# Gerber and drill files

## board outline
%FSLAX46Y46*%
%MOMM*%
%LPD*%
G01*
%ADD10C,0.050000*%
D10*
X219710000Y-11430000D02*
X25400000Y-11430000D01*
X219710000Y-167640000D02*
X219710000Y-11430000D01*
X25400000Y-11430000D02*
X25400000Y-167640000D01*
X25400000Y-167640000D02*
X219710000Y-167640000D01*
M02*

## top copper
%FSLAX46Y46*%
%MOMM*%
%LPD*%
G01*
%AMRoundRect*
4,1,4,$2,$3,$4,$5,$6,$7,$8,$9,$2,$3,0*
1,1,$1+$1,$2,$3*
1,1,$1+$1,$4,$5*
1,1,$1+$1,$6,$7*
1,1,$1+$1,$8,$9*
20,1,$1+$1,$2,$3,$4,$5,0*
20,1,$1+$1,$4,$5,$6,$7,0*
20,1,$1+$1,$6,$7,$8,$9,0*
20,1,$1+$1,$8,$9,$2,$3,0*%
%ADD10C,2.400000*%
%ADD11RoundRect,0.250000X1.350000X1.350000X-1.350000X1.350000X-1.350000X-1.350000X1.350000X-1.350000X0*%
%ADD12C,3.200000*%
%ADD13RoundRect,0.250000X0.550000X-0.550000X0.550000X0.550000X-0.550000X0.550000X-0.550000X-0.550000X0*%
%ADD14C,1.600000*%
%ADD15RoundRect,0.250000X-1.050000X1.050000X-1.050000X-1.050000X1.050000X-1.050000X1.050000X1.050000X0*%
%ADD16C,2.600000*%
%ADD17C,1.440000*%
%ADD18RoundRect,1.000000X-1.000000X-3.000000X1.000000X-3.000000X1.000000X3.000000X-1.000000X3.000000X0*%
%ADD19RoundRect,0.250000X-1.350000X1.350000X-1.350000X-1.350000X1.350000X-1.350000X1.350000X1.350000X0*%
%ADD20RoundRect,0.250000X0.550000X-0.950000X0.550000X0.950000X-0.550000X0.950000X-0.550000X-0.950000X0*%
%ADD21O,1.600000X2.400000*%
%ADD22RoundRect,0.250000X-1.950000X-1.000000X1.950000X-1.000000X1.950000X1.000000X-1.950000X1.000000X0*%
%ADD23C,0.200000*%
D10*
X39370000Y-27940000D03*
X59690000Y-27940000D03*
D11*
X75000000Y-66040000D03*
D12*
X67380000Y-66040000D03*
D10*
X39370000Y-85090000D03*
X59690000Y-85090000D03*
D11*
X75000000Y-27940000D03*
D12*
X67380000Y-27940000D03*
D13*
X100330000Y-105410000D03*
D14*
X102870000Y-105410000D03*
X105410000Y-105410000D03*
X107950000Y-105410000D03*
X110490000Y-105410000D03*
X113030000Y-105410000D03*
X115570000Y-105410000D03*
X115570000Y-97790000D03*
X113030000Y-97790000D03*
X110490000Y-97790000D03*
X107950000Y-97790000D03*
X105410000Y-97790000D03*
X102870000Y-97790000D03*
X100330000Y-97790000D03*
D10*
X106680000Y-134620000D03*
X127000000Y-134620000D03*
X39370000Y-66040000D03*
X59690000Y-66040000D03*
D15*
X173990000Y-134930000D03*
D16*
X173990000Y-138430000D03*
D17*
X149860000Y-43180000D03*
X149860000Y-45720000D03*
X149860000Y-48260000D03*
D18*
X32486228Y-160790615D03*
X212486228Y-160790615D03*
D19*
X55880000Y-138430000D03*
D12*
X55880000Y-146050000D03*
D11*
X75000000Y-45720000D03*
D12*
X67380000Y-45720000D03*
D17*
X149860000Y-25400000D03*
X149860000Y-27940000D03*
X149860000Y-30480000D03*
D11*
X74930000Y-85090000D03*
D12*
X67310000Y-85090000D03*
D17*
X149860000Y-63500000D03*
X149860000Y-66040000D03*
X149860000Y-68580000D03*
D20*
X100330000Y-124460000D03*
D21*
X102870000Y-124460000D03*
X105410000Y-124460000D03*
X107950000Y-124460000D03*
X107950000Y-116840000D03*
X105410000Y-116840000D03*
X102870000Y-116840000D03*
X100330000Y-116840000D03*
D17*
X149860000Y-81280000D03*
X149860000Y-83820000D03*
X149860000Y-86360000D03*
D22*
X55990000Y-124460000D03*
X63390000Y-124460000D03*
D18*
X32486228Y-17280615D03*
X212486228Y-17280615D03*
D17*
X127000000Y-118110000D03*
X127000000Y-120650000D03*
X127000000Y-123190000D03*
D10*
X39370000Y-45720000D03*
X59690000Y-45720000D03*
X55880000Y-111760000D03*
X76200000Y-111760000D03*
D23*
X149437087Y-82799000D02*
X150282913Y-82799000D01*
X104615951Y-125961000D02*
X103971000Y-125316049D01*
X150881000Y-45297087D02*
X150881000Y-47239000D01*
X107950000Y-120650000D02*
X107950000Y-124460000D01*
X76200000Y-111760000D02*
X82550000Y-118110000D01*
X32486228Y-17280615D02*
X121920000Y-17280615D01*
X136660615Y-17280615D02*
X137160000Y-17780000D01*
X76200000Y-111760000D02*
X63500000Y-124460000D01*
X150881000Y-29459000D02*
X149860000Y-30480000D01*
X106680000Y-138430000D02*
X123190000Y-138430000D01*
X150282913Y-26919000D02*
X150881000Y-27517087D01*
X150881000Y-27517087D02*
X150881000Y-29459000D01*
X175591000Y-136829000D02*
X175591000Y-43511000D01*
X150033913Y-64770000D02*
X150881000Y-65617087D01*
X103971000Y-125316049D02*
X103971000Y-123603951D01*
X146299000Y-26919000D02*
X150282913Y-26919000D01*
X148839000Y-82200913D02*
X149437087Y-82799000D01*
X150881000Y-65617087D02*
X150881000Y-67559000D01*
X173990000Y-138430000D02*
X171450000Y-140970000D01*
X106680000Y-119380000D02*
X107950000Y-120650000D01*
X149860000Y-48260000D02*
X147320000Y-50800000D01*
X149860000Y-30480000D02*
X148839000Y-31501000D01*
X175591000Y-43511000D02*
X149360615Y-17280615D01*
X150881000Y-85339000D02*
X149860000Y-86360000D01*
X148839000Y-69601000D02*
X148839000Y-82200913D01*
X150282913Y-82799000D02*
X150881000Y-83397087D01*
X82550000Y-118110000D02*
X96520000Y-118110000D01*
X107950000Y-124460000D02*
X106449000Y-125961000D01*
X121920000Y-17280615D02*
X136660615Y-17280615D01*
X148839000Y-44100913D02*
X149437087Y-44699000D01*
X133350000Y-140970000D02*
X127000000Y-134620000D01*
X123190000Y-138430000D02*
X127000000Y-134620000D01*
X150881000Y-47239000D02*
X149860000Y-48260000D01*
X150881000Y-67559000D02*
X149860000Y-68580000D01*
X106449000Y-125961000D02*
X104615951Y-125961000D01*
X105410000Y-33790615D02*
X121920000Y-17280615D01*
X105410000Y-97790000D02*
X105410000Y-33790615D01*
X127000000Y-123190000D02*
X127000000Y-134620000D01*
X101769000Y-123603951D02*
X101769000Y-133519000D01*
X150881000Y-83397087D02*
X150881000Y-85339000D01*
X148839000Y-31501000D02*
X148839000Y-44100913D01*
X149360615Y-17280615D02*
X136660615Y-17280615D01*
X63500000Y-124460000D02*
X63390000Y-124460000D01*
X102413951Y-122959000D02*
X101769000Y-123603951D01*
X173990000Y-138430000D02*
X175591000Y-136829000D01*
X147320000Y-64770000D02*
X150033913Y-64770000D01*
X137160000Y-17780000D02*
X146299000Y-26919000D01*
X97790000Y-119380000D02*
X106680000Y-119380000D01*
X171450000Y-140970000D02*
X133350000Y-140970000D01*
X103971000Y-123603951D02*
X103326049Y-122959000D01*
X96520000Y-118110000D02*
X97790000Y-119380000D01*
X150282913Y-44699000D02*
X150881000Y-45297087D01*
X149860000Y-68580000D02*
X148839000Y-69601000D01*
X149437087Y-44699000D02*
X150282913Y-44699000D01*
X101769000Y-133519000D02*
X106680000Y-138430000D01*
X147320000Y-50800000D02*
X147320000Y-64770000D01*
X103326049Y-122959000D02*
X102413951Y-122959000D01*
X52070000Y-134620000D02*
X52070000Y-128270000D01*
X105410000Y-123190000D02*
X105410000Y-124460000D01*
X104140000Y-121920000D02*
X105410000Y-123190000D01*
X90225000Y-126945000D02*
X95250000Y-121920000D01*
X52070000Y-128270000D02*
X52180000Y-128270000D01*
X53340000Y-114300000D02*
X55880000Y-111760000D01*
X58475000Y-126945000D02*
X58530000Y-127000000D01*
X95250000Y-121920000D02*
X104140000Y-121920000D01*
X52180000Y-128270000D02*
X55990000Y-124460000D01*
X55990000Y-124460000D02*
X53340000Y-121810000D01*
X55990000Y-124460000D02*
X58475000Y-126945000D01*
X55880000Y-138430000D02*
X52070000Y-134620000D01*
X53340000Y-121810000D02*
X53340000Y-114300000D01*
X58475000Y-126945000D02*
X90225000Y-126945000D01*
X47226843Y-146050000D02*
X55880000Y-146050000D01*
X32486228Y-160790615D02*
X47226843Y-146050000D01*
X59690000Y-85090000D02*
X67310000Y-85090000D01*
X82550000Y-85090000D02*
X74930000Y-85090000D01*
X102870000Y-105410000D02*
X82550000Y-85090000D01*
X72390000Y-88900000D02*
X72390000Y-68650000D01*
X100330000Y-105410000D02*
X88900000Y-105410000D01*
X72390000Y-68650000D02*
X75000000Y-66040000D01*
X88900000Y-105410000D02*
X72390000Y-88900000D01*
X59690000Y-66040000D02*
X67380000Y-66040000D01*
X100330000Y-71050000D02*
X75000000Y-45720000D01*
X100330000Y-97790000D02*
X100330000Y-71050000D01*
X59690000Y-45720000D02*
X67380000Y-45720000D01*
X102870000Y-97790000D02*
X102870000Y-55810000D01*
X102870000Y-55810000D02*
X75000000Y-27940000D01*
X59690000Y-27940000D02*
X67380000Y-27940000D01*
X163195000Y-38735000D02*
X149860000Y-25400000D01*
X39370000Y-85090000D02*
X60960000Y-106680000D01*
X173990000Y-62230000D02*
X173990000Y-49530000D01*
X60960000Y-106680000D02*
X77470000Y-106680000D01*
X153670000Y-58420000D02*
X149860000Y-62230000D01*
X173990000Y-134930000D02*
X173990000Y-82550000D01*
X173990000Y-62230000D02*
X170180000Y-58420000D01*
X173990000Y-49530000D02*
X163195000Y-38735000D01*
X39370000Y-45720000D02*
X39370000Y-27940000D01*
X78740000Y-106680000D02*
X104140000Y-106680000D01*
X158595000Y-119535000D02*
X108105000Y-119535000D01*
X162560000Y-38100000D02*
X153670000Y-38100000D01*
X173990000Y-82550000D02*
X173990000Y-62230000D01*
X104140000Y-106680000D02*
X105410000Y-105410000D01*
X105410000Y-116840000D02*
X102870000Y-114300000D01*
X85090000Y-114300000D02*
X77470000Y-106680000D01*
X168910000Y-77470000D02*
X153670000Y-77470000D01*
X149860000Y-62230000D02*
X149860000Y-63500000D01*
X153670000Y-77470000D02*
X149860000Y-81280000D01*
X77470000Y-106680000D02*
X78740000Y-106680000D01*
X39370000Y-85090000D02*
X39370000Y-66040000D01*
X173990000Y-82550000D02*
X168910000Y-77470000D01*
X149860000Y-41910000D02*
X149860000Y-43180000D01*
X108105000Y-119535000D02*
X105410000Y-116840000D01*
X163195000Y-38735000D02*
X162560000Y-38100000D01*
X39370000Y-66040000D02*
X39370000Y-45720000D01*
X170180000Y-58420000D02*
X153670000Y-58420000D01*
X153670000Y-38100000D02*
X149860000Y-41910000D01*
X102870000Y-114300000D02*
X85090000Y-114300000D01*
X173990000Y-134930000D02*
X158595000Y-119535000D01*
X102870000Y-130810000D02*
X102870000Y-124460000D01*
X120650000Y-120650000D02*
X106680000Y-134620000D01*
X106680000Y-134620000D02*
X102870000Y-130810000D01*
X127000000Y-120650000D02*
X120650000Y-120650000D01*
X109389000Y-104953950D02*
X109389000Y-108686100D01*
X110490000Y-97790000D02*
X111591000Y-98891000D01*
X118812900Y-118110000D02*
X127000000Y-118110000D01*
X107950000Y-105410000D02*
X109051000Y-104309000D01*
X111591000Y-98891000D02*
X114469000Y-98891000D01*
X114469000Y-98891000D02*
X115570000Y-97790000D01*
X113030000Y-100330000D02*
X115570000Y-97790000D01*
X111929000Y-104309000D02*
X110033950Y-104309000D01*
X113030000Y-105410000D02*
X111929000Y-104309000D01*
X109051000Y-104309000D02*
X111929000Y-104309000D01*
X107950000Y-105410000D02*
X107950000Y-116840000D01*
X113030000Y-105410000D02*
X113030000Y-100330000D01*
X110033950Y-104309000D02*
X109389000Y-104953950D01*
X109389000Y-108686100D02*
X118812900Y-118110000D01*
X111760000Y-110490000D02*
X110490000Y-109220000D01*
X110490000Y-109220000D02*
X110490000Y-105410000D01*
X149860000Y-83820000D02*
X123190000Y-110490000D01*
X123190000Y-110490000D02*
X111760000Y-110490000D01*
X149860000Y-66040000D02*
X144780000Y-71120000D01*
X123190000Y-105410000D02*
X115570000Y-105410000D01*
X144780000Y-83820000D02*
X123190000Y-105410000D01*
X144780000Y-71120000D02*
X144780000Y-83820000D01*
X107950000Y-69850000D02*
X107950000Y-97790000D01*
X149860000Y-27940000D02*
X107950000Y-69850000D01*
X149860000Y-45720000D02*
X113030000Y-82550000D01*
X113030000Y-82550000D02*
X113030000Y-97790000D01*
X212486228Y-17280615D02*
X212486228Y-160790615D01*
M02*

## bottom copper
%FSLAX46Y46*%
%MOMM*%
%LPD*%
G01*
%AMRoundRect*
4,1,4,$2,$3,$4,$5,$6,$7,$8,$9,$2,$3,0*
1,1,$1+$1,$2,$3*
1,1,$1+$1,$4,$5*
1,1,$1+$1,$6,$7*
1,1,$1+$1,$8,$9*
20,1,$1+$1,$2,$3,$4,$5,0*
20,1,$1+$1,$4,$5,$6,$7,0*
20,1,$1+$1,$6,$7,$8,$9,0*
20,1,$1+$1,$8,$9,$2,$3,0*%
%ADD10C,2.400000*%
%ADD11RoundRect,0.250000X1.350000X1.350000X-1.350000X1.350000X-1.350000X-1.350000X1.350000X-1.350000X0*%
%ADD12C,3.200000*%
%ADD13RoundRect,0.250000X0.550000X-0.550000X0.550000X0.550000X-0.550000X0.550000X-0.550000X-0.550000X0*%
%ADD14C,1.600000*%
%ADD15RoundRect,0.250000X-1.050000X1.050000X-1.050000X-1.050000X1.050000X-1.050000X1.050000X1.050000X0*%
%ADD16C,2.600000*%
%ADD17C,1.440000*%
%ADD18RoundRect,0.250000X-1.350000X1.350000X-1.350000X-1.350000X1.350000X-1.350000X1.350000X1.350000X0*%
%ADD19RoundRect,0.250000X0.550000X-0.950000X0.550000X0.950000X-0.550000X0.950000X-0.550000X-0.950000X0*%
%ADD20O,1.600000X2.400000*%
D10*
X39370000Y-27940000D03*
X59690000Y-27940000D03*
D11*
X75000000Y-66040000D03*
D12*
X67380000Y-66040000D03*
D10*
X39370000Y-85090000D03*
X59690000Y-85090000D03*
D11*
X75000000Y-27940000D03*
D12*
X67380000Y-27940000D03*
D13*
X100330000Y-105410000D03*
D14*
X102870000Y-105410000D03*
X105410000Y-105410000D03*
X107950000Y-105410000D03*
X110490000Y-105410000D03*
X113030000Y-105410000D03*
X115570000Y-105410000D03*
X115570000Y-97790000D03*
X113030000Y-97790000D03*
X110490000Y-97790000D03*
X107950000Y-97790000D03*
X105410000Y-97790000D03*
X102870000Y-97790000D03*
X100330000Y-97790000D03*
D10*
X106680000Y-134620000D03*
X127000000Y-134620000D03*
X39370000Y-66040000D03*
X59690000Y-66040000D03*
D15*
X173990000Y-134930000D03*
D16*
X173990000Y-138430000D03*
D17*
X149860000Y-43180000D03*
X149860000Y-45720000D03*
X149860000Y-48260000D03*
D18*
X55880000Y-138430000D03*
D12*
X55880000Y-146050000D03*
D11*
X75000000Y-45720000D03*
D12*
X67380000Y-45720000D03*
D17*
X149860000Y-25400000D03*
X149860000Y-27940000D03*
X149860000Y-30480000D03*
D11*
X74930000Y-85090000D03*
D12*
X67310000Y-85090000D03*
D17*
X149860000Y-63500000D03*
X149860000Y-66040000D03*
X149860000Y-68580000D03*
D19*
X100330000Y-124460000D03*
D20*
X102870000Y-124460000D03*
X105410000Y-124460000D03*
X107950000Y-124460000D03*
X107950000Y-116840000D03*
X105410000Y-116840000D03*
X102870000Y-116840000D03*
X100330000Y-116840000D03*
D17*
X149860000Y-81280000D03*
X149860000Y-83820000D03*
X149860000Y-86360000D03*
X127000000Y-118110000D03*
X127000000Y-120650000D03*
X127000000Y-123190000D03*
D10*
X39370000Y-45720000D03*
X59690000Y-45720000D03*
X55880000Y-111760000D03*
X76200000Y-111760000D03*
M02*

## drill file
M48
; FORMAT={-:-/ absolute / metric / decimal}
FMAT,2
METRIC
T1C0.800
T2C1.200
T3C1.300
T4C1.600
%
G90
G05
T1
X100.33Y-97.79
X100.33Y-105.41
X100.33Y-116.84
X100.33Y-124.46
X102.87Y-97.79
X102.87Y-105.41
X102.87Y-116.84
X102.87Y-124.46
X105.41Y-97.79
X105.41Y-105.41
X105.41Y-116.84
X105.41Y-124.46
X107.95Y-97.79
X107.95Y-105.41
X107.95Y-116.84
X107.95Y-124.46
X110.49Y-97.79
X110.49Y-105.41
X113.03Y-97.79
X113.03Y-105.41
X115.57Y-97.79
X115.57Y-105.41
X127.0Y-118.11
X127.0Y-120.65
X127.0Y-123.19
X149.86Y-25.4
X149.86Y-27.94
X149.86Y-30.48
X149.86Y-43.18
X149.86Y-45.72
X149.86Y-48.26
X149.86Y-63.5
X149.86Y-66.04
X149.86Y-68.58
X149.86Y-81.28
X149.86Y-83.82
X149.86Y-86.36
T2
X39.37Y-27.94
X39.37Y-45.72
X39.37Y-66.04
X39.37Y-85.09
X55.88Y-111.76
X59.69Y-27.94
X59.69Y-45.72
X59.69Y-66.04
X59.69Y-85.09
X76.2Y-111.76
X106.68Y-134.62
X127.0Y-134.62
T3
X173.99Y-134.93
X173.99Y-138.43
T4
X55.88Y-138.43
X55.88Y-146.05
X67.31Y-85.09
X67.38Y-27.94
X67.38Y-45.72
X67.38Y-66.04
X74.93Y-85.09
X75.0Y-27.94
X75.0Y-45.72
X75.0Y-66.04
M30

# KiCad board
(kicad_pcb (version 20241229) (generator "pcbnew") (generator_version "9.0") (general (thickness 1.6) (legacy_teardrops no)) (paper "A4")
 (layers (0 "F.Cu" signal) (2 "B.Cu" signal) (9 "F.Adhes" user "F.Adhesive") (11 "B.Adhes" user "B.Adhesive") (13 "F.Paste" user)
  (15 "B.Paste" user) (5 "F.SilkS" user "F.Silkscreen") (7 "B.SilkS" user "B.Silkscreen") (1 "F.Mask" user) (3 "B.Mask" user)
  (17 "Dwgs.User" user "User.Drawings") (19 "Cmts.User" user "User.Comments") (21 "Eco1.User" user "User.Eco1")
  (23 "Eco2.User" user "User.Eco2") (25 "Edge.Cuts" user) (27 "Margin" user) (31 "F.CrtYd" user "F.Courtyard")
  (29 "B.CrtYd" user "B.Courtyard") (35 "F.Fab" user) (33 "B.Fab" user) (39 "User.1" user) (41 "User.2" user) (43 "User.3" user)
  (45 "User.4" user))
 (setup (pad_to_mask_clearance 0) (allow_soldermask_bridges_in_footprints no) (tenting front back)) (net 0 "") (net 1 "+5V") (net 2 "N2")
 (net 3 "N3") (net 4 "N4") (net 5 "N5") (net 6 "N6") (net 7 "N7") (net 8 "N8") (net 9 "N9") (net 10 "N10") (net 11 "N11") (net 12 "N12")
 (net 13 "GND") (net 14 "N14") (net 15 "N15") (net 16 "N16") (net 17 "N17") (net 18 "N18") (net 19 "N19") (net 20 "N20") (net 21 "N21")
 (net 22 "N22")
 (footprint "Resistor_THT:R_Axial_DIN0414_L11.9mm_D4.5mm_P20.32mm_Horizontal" (layer "F.Cu") (at 39.37 27.94)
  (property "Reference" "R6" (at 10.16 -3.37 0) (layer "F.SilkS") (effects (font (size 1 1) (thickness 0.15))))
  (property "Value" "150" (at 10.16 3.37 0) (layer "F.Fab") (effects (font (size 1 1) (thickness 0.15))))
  (pad "1" thru_hole circle (at 0 0) (size 2.4 2.4) (drill 1.2) (layers "*.Cu" "*.Mask") (remove_unused_layers no) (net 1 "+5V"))
  (pad "2" thru_hole circle (at 20.32 0) (size 2.4 2.4) (drill 1.2) (layers "*.Cu" "*.Mask") (remove_unused_layers no) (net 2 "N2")))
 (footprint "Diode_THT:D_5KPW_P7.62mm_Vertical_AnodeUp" (layer "F.Cu") (at 75 66.04 180)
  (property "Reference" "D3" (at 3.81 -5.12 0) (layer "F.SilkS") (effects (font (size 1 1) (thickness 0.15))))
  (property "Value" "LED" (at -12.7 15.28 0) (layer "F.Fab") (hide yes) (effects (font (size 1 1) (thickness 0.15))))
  (pad "1" thru_hole roundrect (at 0 0 180) (size 3.2 3.2) (drill 1.6) (layers "*.Cu" "*.Mask") (remove_unused_layers no)
   (roundrect_rratio 0.078125) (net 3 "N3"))
  (pad "2" thru_hole circle (at 7.62 0 180) (size 3.2 3.2) (drill 1.6) (layers "*.Cu" "*.Mask") (remove_unused_layers no) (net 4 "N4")))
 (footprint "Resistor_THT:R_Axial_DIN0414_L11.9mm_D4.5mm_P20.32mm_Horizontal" (layer "F.Cu") (at 39.37 85.09)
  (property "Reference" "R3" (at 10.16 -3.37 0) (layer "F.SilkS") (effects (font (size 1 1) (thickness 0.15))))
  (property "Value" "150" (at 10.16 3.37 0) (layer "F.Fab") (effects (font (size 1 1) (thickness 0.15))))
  (pad "1" thru_hole circle (at 0 0) (size 2.4 2.4) (drill 1.2) (layers "*.Cu" "*.Mask") (remove_unused_layers no) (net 1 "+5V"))
  (pad "2" thru_hole circle (at 20.32 0) (size 2.4 2.4) (drill 1.2) (layers "*.Cu" "*.Mask") (remove_unused_layers no) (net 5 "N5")))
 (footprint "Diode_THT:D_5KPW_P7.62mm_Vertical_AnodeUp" (layer "F.Cu") (at 75 27.94 180)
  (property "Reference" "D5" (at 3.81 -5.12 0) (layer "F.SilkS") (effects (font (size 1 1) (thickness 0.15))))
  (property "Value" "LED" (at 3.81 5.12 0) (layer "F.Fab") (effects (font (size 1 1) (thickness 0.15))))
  (pad "1" thru_hole roundrect (at 0 0 180) (size 3.2 3.2) (drill 1.6) (layers "*.Cu" "*.Mask") (remove_unused_layers no)
   (roundrect_rratio 0.078125) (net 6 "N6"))
  (pad "2" thru_hole circle (at 7.62 0 180) (size 3.2 3.2) (drill 1.6) (layers "*.Cu" "*.Mask") (remove_unused_layers no) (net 2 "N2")))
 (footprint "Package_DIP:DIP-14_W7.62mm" (layer "F.Cu") (at 100.33 105.41 90)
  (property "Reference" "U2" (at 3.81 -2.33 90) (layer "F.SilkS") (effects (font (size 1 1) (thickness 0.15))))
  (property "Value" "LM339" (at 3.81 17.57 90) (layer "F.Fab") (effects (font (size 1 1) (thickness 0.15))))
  (pad "1" thru_hole roundrect (at 0 0 90) (size 1.6 1.6) (drill 0.8) (layers "*.Cu" "*.Mask") (remove_unused_layers no)
   (roundrect_rratio 0.15625) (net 3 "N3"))
  (pad "2" thru_hole circle (at 0 2.54 90) (size 1.6 1.6) (drill 0.8) (layers "*.Cu" "*.Mask") (remove_unused_layers no) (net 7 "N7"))
  (pad "3" thru_hole circle (at 0 5.08 90) (size 1.6 1.6) (drill 0.8) (layers "*.Cu" "*.Mask") (remove_unused_layers no) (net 1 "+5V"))
  (pad "4" thru_hole circle (at 0 7.62 90) (size 1.6 1.6) (drill 0.8) (layers "*.Cu" "*.Mask") (remove_unused_layers no) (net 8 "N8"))
  (pad "5" thru_hole circle (at 0 10.16 90) (size 1.6 1.6) (drill 0.8) (layers "*.Cu" "*.Mask") (remove_unused_layers no) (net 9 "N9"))
  (pad "6" thru_hole circle (at 0 12.7 90) (size 1.6 1.6) (drill 0.8) (layers "*.Cu" "*.Mask") (remove_unused_layers no) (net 8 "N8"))
  (pad "7" thru_hole circle (at 0 15.24 90) (size 1.6 1.6) (drill 0.8) (layers "*.Cu" "*.Mask") (remove_unused_layers no) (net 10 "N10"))
  (pad "8" thru_hole circle (at 7.62 15.24 90) (size 1.6 1.6) (drill 0.8) (layers "*.Cu" "*.Mask") (remove_unused_layers no) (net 8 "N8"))
  (pad "9" thru_hole circle (at 7.62 12.7 90) (size 1.6 1.6) (drill 0.8) (layers "*.Cu" "*.Mask") (remove_unused_layers no) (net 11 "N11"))
  (pad "10" thru_hole circle (at 7.62 10.16 90) (size 1.6 1.6) (drill 0.8) (layers "*.Cu" "*.Mask") (remove_unused_layers no) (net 8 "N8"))
  (pad "11" thru_hole circle (at 7.62 7.62 90) (size 1.6 1.6) (drill 0.8) (layers "*.Cu" "*.Mask") (remove_unused_layers no) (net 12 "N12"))
  (pad "12" thru_hole circle (at 7.62 5.08 90) (size 1.6 1.6) (drill 0.8) (layers "*.Cu" "*.Mask") (remove_unused_layers no) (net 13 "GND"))
  (pad "13" thru_hole circle (at 7.62 2.54 90) (size 1.6 1.6) (drill 0.8) (layers "*.Cu" "*.Mask") (remove_unused_layers no) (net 6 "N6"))
  (pad "14" thru_hole circle (at 7.62 0 90) (size 1.6 1.6) (drill 0.8) (layers "*.Cu" "*.Mask") (remove_unused_layers no) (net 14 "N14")))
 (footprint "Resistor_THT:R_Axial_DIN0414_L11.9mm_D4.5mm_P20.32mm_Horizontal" (layer "F.Cu") (at 106.68 134.62)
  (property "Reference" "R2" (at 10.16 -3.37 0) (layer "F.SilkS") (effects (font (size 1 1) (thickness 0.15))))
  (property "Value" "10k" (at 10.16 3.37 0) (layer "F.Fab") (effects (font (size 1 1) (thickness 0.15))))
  (pad "1" thru_hole circle (at 0 0) (size 2.4 2.4) (drill 1.2) (layers "*.Cu" "*.Mask") (remove_unused_layers no) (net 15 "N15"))
  (pad "2" thru_hole circle (at 20.32 0) (size 2.4 2.4) (drill 1.2) (layers "*.Cu" "*.Mask") (remove_unused_layers no) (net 13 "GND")))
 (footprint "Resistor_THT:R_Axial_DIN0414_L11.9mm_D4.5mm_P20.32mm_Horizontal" (layer "F.Cu") (at 39.37 66.04)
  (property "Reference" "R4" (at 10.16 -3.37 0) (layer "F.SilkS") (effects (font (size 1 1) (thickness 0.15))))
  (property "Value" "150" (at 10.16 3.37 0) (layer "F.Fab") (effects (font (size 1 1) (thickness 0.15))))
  (pad "1" thru_hole circle (at 0 0) (size 2.4 2.4) (drill 1.2) (layers "*.Cu" "*.Mask") (remove_unused_layers no) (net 1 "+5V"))
  (pad "2" thru_hole circle (at 20.32 0) (size 2.4 2.4) (drill 1.2) (layers "*.Cu" "*.Mask") (remove_unused_layers no) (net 4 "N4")))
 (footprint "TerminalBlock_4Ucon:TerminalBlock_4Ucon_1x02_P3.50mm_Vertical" (layer "F.Cu") (at 173.99 134.93 -90)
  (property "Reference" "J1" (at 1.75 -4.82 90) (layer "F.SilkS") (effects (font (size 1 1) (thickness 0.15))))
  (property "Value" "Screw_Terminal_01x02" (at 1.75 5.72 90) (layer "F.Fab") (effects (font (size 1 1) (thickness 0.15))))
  (pad "1" thru_hole roundrect (at 0 0 270) (size 2.6 2.6) (drill 1.3) (layers "*.Cu" "*.Mask") (remove_unused_layers no)
   (roundrect_rratio 0.096154) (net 1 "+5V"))
  (pad "2" thru_hole circle (at 3.5 0 270) (size 2.6 2.6) (drill 1.3) (layers "*.Cu" "*.Mask") (remove_unused_layers no) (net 13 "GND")))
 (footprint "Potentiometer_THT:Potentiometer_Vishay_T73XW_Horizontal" (layer "F.Cu") (at 149.86 43.18)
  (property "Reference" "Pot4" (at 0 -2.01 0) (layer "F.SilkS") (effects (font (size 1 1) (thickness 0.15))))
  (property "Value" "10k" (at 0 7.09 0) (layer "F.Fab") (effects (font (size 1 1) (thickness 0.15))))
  (pad "1" thru_hole circle (at 0 0) (size 1.44 1.44) (drill 0.8) (layers "*.Cu" "*.Mask") (remove_unused_layers no) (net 1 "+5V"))
  (pad "2" thru_hole circle (at 0 2.54) (size 1.44 1.44) (drill 0.8) (layers "*.Cu" "*.Mask") (remove_unused_layers no) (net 11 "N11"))
  (pad "3" thru_hole circle (at 0 5.08) (size 1.44 1.44) (drill 0.8) (layers "*.Cu" "*.Mask") (remove_unused_layers no) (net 13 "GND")))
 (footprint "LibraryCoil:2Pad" (layer "F.Cu") (at 32.486228 160.790615 90)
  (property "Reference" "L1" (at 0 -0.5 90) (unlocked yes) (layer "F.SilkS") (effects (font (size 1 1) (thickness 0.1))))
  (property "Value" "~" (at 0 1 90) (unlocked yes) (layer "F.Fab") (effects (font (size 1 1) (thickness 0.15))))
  (pad "1" smd roundrect (at 0 0) (size 4 8) (layers "F.Cu" "F.Mask") (roundrect_rratio 0.25) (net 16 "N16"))
  (pad "2" smd roundrect (at 0 180) (size 4 8) (layers "F.Cu" "F.Mask") (roundrect_rratio 0.25) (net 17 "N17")))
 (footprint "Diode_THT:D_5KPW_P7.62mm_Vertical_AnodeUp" (layer "F.Cu") (at 55.88 138.43 -90)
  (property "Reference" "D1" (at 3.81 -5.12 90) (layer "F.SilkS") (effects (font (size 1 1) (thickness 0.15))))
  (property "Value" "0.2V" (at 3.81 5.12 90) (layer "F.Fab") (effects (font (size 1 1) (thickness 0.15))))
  (pad "1" thru_hole roundrect (at 0 0 270) (size 3.2 3.2) (drill 1.6) (layers "*.Cu" "*.Mask") (remove_unused_layers no)
   (roundrect_rratio 0.078125) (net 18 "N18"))
  (pad "2" thru_hole circle (at 7.62 0 270) (size 3.2 3.2) (drill 1.6) (layers "*.Cu" "*.Mask") (remove_unused_layers no) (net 16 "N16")))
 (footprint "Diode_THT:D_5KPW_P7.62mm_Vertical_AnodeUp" (layer "F.Cu") (at 75 45.72 180)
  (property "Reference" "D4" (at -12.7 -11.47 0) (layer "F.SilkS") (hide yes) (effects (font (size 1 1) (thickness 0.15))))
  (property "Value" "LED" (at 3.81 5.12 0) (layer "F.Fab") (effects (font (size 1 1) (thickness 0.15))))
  (pad "1" thru_hole roundrect (at 0 0 180) (size 3.2 3.2) (drill 1.6) (layers "*.Cu" "*.Mask") (remove_unused_layers no)
   (roundrect_rratio 0.078125) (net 14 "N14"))
  (pad "2" thru_hole circle (at 7.62 0 180) (size 3.2 3.2) (drill 1.6) (layers "*.Cu" "*.Mask") (remove_unused_layers no) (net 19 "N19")))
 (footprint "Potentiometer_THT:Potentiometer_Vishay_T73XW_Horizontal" (layer "F.Cu") (at 149.86 25.4)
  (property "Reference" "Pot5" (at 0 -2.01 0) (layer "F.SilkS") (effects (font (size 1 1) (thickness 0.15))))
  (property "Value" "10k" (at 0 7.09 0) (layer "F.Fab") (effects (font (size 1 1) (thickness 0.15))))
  (pad "1" thru_hole circle (at 0 0) (size 1.44 1.44) (drill 0.8) (layers "*.Cu" "*.Mask") (remove_unused_layers no) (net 1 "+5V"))
  (pad "2" thru_hole circle (at 0 2.54) (size 1.44 1.44) (drill 0.8) (layers "*.Cu" "*.Mask") (remove_unused_layers no) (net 12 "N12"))
  (pad "3" thru_hole circle (at 0 5.08) (size 1.44 1.44) (drill 0.8) (layers "*.Cu" "*.Mask") (remove_unused_layers no) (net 13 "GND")))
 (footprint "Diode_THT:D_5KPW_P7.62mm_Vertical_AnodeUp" (layer "F.Cu") (at 74.93 85.09 180)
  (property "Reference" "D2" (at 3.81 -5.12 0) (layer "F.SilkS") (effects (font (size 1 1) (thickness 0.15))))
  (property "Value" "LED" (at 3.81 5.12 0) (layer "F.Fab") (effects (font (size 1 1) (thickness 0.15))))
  (pad "1" thru_hole roundrect (at 0 0 180) (size 3.2 3.2) (drill 1.6) (layers "*.Cu" "*.Mask") (remove_unused_layers no)
   (roundrect_rratio 0.078125) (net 7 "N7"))
  (pad "2" thru_hole circle (at 7.62 0 180) (size 3.2 3.2) (drill 1.6) (layers "*.Cu" "*.Mask") (remove_unused_layers no) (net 5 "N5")))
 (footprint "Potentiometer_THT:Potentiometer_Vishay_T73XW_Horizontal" (layer "F.Cu") (at 149.86 63.5)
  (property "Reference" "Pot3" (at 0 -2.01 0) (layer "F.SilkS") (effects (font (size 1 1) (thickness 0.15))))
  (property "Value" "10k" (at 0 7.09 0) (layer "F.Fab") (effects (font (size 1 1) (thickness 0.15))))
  (pad "1" thru_hole circle (at 0 0) (size 1.44 1.44) (drill 0.8) (layers "*.Cu" "*.Mask") (remove_unused_layers no) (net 1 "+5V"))
  (pad "2" thru_hole circle (at 0 2.54) (size 1.44 1.44) (drill 0.8) (layers "*.Cu" "*.Mask") (remove_unused_layers no) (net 10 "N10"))
  (pad "3" thru_hole circle (at 0 5.08) (size 1.44 1.44) (drill 0.8) (layers "*.Cu" "*.Mask") (remove_unused_layers no) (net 13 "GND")))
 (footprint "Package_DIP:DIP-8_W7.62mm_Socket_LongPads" (layer "F.Cu") (at 100.33 124.46 90)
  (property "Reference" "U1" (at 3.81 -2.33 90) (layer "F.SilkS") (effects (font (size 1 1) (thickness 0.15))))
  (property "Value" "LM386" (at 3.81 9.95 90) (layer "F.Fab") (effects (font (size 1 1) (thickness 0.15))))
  (pad "1" thru_hole roundrect (at 0 0 90) (size 2.4 1.6) (drill 0.8) (layers "*.Cu" "*.Mask") (remove_unused_layers no)
   (roundrect_rratio 0.15625) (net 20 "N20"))
  (pad "2" thru_hole oval (at 0 2.54 90) (size 2.4 1.6) (drill 0.8) (layers "*.Cu" "*.Mask") (remove_unused_layers no) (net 15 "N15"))
  (pad "3" thru_hole oval (at 0 5.08 90) (size 2.4 1.6) (drill 0.8) (layers "*.Cu" "*.Mask") (remove_unused_layers no) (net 18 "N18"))
  (pad "4" thru_hole oval (at 0 7.62 90) (size 2.4 1.6) (drill 0.8) (layers "*.Cu" "*.Mask") (remove_unused_layers no) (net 13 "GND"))
  (pad "5" thru_hole oval (at 7.62 7.62 90) (size 2.4 1.6) (drill 0.8) (layers "*.Cu" "*.Mask") (remove_unused_layers no) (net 8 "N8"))
  (pad "6" thru_hole oval (at 7.62 5.08 90) (size 2.4 1.6) (drill 0.8) (layers "*.Cu" "*.Mask") (remove_unused_layers no) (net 1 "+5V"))
  (pad "7" thru_hole oval (at 7.62 2.54 90) (size 2.4 1.6) (drill 0.8) (layers "*.Cu" "*.Mask") (remove_unused_layers no) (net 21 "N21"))
  (pad "8" thru_hole oval (at 7.62 0 90) (size 2.4 1.6) (drill 0.8) (layers "*.Cu" "*.Mask") (remove_unused_layers no) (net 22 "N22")))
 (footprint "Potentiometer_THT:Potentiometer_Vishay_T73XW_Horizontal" (layer "F.Cu") (at 149.86 81.28)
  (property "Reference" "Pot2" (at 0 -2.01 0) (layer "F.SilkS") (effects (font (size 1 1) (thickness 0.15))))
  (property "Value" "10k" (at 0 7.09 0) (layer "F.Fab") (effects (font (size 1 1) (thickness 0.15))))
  (pad "1" thru_hole circle (at 0 0) (size 1.44 1.44) (drill 0.8) (layers "*.Cu" "*.Mask") (remove_unused_layers no) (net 1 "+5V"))
  (pad "2" thru_hole circle (at 0 2.54) (size 1.44 1.44) (drill 0.8) (layers "*.Cu" "*.Mask") (remove_unused_layers no) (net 9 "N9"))
  (pad "3" thru_hole circle (at 0 5.08) (size 1.44 1.44) (drill 0.8) (layers "*.Cu" "*.Mask") (remove_unused_layers no) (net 13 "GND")))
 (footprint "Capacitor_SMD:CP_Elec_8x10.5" (layer "F.Cu") (at 59.69 124.46)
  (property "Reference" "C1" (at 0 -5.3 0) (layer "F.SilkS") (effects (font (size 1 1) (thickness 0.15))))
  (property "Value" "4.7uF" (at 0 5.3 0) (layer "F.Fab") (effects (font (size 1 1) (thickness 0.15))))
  (pad "1" smd roundrect (at -3.7 0) (size 4.4 2.5) (layers "F.Cu" "F.Mask" "F.Paste") (roundrect_rratio 0.1) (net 18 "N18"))
  (pad "2" smd roundrect (at 3.7 0) (size 4.4 2.5) (layers "F.Cu" "F.Mask" "F.Paste") (roundrect_rratio 0.1) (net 13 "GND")))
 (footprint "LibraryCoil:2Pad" (layer "F.Cu") (at 32.486228 17.280615 90)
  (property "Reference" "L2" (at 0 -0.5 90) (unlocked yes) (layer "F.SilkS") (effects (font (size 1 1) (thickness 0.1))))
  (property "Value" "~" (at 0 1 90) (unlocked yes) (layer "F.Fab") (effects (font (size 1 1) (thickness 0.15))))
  (pad "1" smd roundrect (at 0 0) (size 4 8) (layers "F.Cu" "F.Mask") (roundrect_rratio 0.25) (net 13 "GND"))
  (pad "2" smd roundrect (at 0 180) (size 4 8) (layers "F.Cu" "F.Mask") (roundrect_rratio 0.25) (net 17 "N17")))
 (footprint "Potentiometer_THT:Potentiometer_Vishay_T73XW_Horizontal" (layer "F.Cu") (at 127 118.11)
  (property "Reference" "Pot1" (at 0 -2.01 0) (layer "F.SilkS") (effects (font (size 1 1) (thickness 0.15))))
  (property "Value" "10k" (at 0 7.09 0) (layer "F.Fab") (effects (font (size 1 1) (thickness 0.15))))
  (pad "1" thru_hole circle (at 0 0) (size 1.44 1.44) (drill 0.8) (layers "*.Cu" "*.Mask") (remove_unused_layers no) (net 8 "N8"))
  (pad "2" thru_hole circle (at 0 2.54) (size 1.44 1.44) (drill 0.8) (layers "*.Cu" "*.Mask") (remove_unused_layers no) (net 15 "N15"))
  (pad "3" thru_hole circle (at 0 5.08) (size 1.44 1.44) (drill 0.8) (layers "*.Cu" "*.Mask") (remove_unused_layers no) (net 13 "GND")))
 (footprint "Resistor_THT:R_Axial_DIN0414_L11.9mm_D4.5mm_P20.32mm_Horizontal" (layer "F.Cu") (at 39.37 45.72)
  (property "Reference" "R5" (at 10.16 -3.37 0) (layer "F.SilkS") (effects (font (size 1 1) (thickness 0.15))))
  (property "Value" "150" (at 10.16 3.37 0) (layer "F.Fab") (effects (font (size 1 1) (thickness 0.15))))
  (pad "1" thru_hole circle (at 0 0) (size 2.4 2.4) (drill 1.2) (layers "*.Cu" "*.Mask") (remove_unused_layers no) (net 1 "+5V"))
  (pad "2" thru_hole circle (at 20.32 0) (size 2.4 2.4) (drill 1.2) (layers "*.Cu" "*.Mask") (remove_unused_layers no) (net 19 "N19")))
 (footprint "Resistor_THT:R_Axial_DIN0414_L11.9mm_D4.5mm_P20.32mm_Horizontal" (layer "F.Cu") (at 55.88 111.76)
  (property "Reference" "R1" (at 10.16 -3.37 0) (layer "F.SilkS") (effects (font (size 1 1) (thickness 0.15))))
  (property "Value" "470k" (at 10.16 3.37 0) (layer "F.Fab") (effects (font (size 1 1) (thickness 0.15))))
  (pad "1" thru_hole circle (at 0 0) (size 2.4 2.4) (drill 1.2) (layers "*.Cu" "*.Mask") (remove_unused_layers no) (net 18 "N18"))
  (pad "2" thru_hole circle (at 20.32 0) (size 2.4 2.4) (drill 1.2) (layers "*.Cu" "*.Mask") (remove_unused_layers no) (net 13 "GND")))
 (gr_line (start 219.71 11.43) (end 25.4 11.43) (stroke (width 0.05) (type default)) (layer "Edge.Cuts"))
 (gr_line (start 219.71 167.64) (end 219.71 11.43) (stroke (width 0.05) (type default)) (layer "Edge.Cuts"))
 (gr_line (start 25.4 11.43) (end 25.4 167.64) (stroke (width 0.05) (type default)) (layer "Edge.Cuts"))
 (gr_line (start 25.4 167.64) (end 219.71 167.64) (stroke (width 0.05) (type default)) (layer "Edge.Cuts"))
 (segment (start 149.437087 82.799) (end 150.282913 82.799) (width 0.2) (layer "F.Cu") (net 13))
 (segment (start 104.615951 125.961) (end 103.971 125.316049) (width 0.2) (layer "F.Cu") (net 13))
 (segment (start 150.881 45.297087) (end 150.881 47.239) (width 0.2) (layer "F.Cu") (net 13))
 (segment (start 107.95 120.65) (end 107.95 124.46) (width 0.2) (layer "F.Cu") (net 13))
 (segment (start 76.2 111.76) (end 82.55 118.11) (width 0.2) (layer "F.Cu") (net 13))
 (segment (start 32.486228 17.280615) (end 121.92 17.280615) (width 0.2) (layer "F.Cu") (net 13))
 (segment (start 136.660615 17.280615) (end 137.16 17.78) (width 0.2) (layer "F.Cu") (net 13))
 (segment (start 76.2 111.76) (end 63.5 124.46) (width 0.2) (layer "F.Cu") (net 13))
 (segment (start 150.881 29.459) (end 149.86 30.48) (width 0.2) (layer "F.Cu") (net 13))
 (segment (start 106.68 138.43) (end 123.19 138.43) (width 0.2) (layer "F.Cu") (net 13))
 (segment (start 150.282913 26.919) (end 150.881 27.517087) (width 0.2) (layer "F.Cu") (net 13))
 (segment (start 150.881 27.517087) (end 150.881 29.459) (width 0.2) (layer "F.Cu") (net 13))
 (segment (start 175.591 136.829) (end 175.591 43.511) (width 0.2) (layer "F.Cu") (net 13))
 (segment (start 150.033913 64.77) (end 150.881 65.617087) (width 0.2) (layer "F.Cu") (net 13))
 (segment (start 103.971 125.316049) (end 103.971 123.603951) (width 0.2) (layer "F.Cu") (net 13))
 (segment (start 146.299 26.919) (end 150.282913 26.919) (width 0.2) (layer "F.Cu") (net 13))
 (segment (start 148.839 82.200913) (end 149.437087 82.799) (width 0.2) (layer "F.Cu") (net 13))
 (segment (start 150.881 65.617087) (end 150.881 67.559) (width 0.2) (layer "F.Cu") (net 13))
 (segment (start 173.99 138.43) (end 171.45 140.97) (width 0.2) (layer "F.Cu") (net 13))
 (segment (start 106.68 119.38) (end 107.95 120.65) (width 0.2) (layer "F.Cu") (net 13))
 (segment (start 149.86 48.26) (end 147.32 50.8) (width 0.2) (layer "F.Cu") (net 13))
 (segment (start 149.86 30.48) (end 148.839 31.501) (width 0.2) (layer "F.Cu") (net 13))
 (segment (start 175.591 43.511) (end 149.360615 17.280615) (width 0.2) (layer "F.Cu") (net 13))
 (segment (start 150.881 85.339) (end 149.86 86.36) (width 0.2) (layer "F.Cu") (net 13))
 (segment (start 148.839 69.601) (end 148.839 82.200913) (width 0.2) (layer "F.Cu") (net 13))
 (segment (start 150.282913 82.799) (end 150.881 83.397087) (width 0.2) (layer "F.Cu") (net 13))
 (segment (start 82.55 118.11) (end 96.52 118.11) (width 0.2) (layer "F.Cu") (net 13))
 (segment (start 107.95 124.46) (end 106.449 125.961) (width 0.2) (layer "F.Cu") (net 13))
 (segment (start 121.92 17.280615) (end 136.660615 17.280615) (width 0.2) (layer "F.Cu") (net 13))
 (segment (start 148.839 44.100913) (end 149.437087 44.699) (width 0.2) (layer "F.Cu") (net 13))
 (segment (start 133.35 140.97) (end 127 134.62) (width 0.2) (layer "F.Cu") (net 13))
 (segment (start 123.19 138.43) (end 127 134.62) (width 0.2) (layer "F.Cu") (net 13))
 (segment (start 150.881 47.239) (end 149.86 48.26) (width 0.2) (layer "F.Cu") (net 13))
 (segment (start 150.881 67.559) (end 149.86 68.58) (width 0.2) (layer "F.Cu") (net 13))
 (segment (start 106.449 125.961) (end 104.615951 125.961) (width 0.2) (layer "F.Cu") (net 13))
 (segment (start 105.41 33.790615) (end 121.92 17.280615) (width 0.2) (layer "F.Cu") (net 13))
 (segment (start 105.41 97.79) (end 105.41 33.790615) (width 0.2) (layer "F.Cu") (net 13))
 (segment (start 127 123.19) (end 127 134.62) (width 0.2) (layer "F.Cu") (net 13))
 (segment (start 101.769 123.603951) (end 101.769 133.519) (width 0.2) (layer "F.Cu") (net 13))
 (segment (start 150.881 83.397087) (end 150.881 85.339) (width 0.2) (layer "F.Cu") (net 13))
 (segment (start 148.839 31.501) (end 148.839 44.100913) (width 0.2) (layer "F.Cu") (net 13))
 (segment (start 149.360615 17.280615) (end 136.660615 17.280615) (width 0.2) (layer "F.Cu") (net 13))
 (segment (start 63.5 124.46) (end 63.39 124.46) (width 0.2) (layer "F.Cu") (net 13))
 (segment (start 102.413951 122.959) (end 101.769 123.603951) (width 0.2) (layer "F.Cu") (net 13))
 (segment (start 173.99 138.43) (end 175.591 136.829) (width 0.2) (layer "F.Cu") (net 13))
 (segment (start 147.32 64.77) (end 150.033913 64.77) (width 0.2) (layer "F.Cu") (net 13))
 (segment (start 137.16 17.78) (end 146.299 26.919) (width 0.2) (layer "F.Cu") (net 13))
 (segment (start 97.79 119.38) (end 106.68 119.38) (width 0.2) (layer "F.Cu") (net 13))
 (segment (start 171.45 140.97) (end 133.35 140.97) (width 0.2) (layer "F.Cu") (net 13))
 (segment (start 103.971 123.603951) (end 103.326049 122.959) (width 0.2) (layer "F.Cu") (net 13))
 (segment (start 96.52 118.11) (end 97.79 119.38) (width 0.2) (layer "F.Cu") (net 13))
 (segment (start 150.282913 44.699) (end 150.881 45.297087) (width 0.2) (layer "F.Cu") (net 13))
 (segment (start 149.86 68.58) (end 148.839 69.601) (width 0.2) (layer "F.Cu") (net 13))
 (segment (start 149.437087 44.699) (end 150.282913 44.699) (width 0.2) (layer "F.Cu") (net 13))
 (segment (start 101.769 133.519) (end 106.68 138.43) (width 0.2) (layer "F.Cu") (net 13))
 (segment (start 147.32 50.8) (end 147.32 64.77) (width 0.2) (layer "F.Cu") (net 13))
 (segment (start 103.326049 122.959) (end 102.413951 122.959) (width 0.2) (layer "F.Cu") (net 13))
 (segment (start 52.07 134.62) (end 52.07 128.27) (width 0.2) (layer "F.Cu") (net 18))
 (segment (start 105.41 123.19) (end 105.41 124.46) (width 0.2) (layer "F.Cu") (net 18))
 (segment (start 104.14 121.92) (end 105.41 123.19) (width 0.2) (layer "F.Cu") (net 18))
 (segment (start 90.225 126.945) (end 95.25 121.92) (width 0.2) (layer "F.Cu") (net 18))
 (segment (start 52.07 128.27) (end 52.18 128.27) (width 0.2) (layer "F.Cu") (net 18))
 (segment (start 53.34 114.3) (end 55.88 111.76) (width 0.2) (layer "F.Cu") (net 18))
 (segment (start 58.475 126.945) (end 58.53 127) (width 0.2) (layer "F.Cu") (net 18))
 (segment (start 95.25 121.92) (end 104.14 121.92) (width 0.2) (layer "F.Cu") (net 18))
 (segment (start 52.18 128.27) (end 55.99 124.46) (width 0.2) (layer "F.Cu") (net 18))
 (segment (start 55.99 124.46) (end 53.34 121.81) (width 0.2) (layer "F.Cu") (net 18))
 (segment (start 55.99 124.46) (end 58.475 126.945) (width 0.2) (layer "F.Cu") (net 18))
 (segment (start 55.88 138.43) (end 52.07 134.62) (width 0.2) (layer "F.Cu") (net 18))
 (segment (start 53.34 121.81) (end 53.34 114.3) (width 0.2) (layer "F.Cu") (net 18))
 (segment (start 58.475 126.945) (end 90.225 126.945) (width 0.2) (layer "F.Cu") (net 18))
 (segment (start 47.226843 146.05) (end 55.88 146.05) (width 0.2) (layer "F.Cu") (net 16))
 (segment (start 32.486228 160.790615) (end 47.226843 146.05) (width 0.2) (layer "F.Cu") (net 16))
 (segment (start 59.69 85.09) (end 67.31 85.09) (width 0.2) (layer "F.Cu") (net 5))
 (segment (start 82.55 85.09) (end 74.93 85.09) (width 0.2) (layer "F.Cu") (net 7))
 (segment (start 102.87 105.41) (end 82.55 85.09) (width 0.2) (layer "F.Cu") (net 7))
 (segment (start 72.39 88.9) (end 72.39 68.65) (width 0.2) (layer "F.Cu") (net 3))
 (segment (start 100.33 105.41) (end 88.9 105.41) (width 0.2) (layer "F.Cu") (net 3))
 (segment (start 72.39 68.65) (end 75 66.04) (width 0.2) (layer "F.Cu") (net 3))
 (segment (start 88.9 105.41) (end 72.39 88.9) (width 0.2) (layer "F.Cu") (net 3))
 (segment (start 59.69 66.04) (end 67.38 66.04) (width 0.2) (layer "F.Cu") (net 4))
 (segment (start 100.33 71.05) (end 75 45.72) (width 0.2) (layer "F.Cu") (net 14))
 (segment (start 100.33 97.79) (end 100.33 71.05) (width 0.2) (layer "F.Cu") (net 14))
 (segment (start 59.69 45.72) (end 67.38 45.72) (width 0.2) (layer "F.Cu") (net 19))
 (segment (start 102.87 97.79) (end 102.87 55.81) (width 0.2) (layer "F.Cu") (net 6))
 (segment (start 102.87 55.81) (end 75 27.94) (width 0.2) (layer "F.Cu") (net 6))
 (segment (start 59.69 27.94) (end 67.38 27.94) (width 0.2) (layer "F.Cu") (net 2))
 (segment (start 163.195 38.735) (end 149.86 25.4) (width 0.2) (layer "F.Cu") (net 1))
 (segment (start 39.37 85.09) (end 60.96 106.68) (width 0.2) (layer "F.Cu") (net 1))
 (segment (start 173.99 62.23) (end 173.99 49.53) (width 0.2) (layer "F.Cu") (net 1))
 (segment (start 60.96 106.68) (end 77.47 106.68) (width 0.2) (layer "F.Cu") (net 1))
 (segment (start 153.67 58.42) (end 149.86 62.23) (width 0.2) (layer "F.Cu") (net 1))
 (segment (start 173.99 134.93) (end 173.99 82.55) (width 0.2) (layer "F.Cu") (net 1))
 (segment (start 173.99 62.23) (end 170.18 58.42) (width 0.2) (layer "F.Cu") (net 1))
 (segment (start 173.99 49.53) (end 163.195 38.735) (width 0.2) (layer "F.Cu") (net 1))
 (segment (start 39.37 45.72) (end 39.37 27.94) (width 0.2) (layer "F.Cu") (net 1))
 (segment (start 78.74 106.68) (end 104.14 106.68) (width 0.2) (layer "F.Cu") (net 1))
 (segment (start 158.595 119.535) (end 108.105 119.535) (width 0.2) (layer "F.Cu") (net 1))
 (segment (start 162.56 38.1) (end 153.67 38.1) (width 0.2) (layer "F.Cu") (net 1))
 (segment (start 173.99 82.55) (end 173.99 62.23) (width 0.2) (layer "F.Cu") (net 1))
 (segment (start 104.14 106.68) (end 105.41 105.41) (width 0.2) (layer "F.Cu") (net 1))
 (segment (start 105.41 116.84) (end 102.87 114.3) (width 0.2) (layer "F.Cu") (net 1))
 (segment (start 85.09 114.3) (end 77.47 106.68) (width 0.2) (layer "F.Cu") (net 1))
 (segment (start 168.91 77.47) (end 153.67 77.47) (width 0.2) (layer "F.Cu") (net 1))
 (segment (start 149.86 62.23) (end 149.86 63.5) (width 0.2) (layer "F.Cu") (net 1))
 (segment (start 153.67 77.47) (end 149.86 81.28) (width 0.2) (layer "F.Cu") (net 1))
 (segment (start 77.47 106.68) (end 78.74 106.68) (width 0.2) (layer "F.Cu") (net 1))
 (segment (start 39.37 85.09) (end 39.37 66.04) (width 0.2) (layer "F.Cu") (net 1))
 (segment (start 173.99 82.55) (end 168.91 77.47) (width 0.2) (layer "F.Cu") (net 1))
 (segment (start 149.86 41.91) (end 149.86 43.18) (width 0.2) (layer "F.Cu") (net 1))
 (segment (start 108.105 119.535) (end 105.41 116.84) (width 0.2) (layer "F.Cu") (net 1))
 (segment (start 163.195 38.735) (end 162.56 38.1) (width 0.2) (layer "F.Cu") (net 1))
 (segment (start 39.37 66.04) (end 39.37 45.72) (width 0.2) (layer "F.Cu") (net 1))
 (segment (start 170.18 58.42) (end 153.67 58.42) (width 0.2) (layer "F.Cu") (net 1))
 (segment (start 153.67 38.1) (end 149.86 41.91) (width 0.2) (layer "F.Cu") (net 1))
 (segment (start 102.87 114.3) (end 85.09 114.3) (width 0.2) (layer "F.Cu") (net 1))
 (segment (start 173.99 134.93) (end 158.595 119.535) (width 0.2) (layer "F.Cu") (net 1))
 (segment (start 102.87 130.81) (end 102.87 124.46) (width 0.2) (layer "F.Cu") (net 15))
 (segment (start 120.65 120.65) (end 106.68 134.62) (width 0.2) (layer "F.Cu") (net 15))
 (segment (start 106.68 134.62) (end 102.87 130.81) (width 0.2) (layer "F.Cu") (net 15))
 (segment (start 127 120.65) (end 120.65 120.65) (width 0.2) (layer "F.Cu") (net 15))
 (segment (start 109.389 104.95395) (end 109.389 108.6861) (width 0.2) (layer "F.Cu") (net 8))
 (segment (start 110.49 97.79) (end 111.591 98.891) (width 0.2) (layer "F.Cu") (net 8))
 (segment (start 118.8129 118.11) (end 127 118.11) (width 0.2) (layer "F.Cu") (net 8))
 (segment (start 107.95 105.41) (end 109.051 104.309) (width 0.2) (layer "F.Cu") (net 8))
 (segment (start 111.591 98.891) (end 114.469 98.891) (width 0.2) (layer "F.Cu") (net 8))
 (segment (start 114.469 98.891) (end 115.57 97.79) (width 0.2) (layer "F.Cu") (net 8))
 (segment (start 113.03 100.33) (end 115.57 97.79) (width 0.2) (layer "F.Cu") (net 8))
 (segment (start 111.929 104.309) (end 110.03395 104.309) (width 0.2) (layer "F.Cu") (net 8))
 (segment (start 113.03 105.41) (end 111.929 104.309) (width 0.2) (layer "F.Cu") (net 8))
 (segment (start 109.051 104.309) (end 111.929 104.309) (width 0.2) (layer "F.Cu") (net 8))
 (segment (start 107.95 105.41) (end 107.95 116.84) (width 0.2) (layer "F.Cu") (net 8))
 (segment (start 113.03 105.41) (end 113.03 100.33) (width 0.2) (layer "F.Cu") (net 8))
 (segment (start 110.03395 104.309) (end 109.389 104.95395) (width 0.2) (layer "F.Cu") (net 8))
 (segment (start 109.389 108.6861) (end 118.8129 118.11) (width 0.2) (layer "F.Cu") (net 8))
 (segment (start 111.76 110.49) (end 110.49 109.22) (width 0.2) (layer "F.Cu") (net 9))
 (segment (start 110.49 109.22) (end 110.49 105.41) (width 0.2) (layer "F.Cu") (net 9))
 (segment (start 149.86 83.82) (end 123.19 110.49) (width 0.2) (layer "F.Cu") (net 9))
 (segment (start 123.19 110.49) (end 111.76 110.49) (width 0.2) (layer "F.Cu") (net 9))
 (segment (start 149.86 66.04) (end 144.78 71.12) (width 0.2) (layer "F.Cu") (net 10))
 (segment (start 123.19 105.41) (end 115.57 105.41) (width 0.2) (layer "F.Cu") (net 10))
 (segment (start 144.78 83.82) (end 123.19 105.41) (width 0.2) (layer "F.Cu") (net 10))
 (segment (start 144.78 71.12) (end 144.78 83.82) (width 0.2) (layer "F.Cu") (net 10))
 (segment (start 107.95 69.85) (end 107.95 97.79) (width 0.2) (layer "F.Cu") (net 12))
 (segment (start 149.86 27.94) (end 107.95 69.85) (width 0.2) (layer "F.Cu") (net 12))
 (segment (start 149.86 45.72) (end 113.03 82.55) (width 0.2) (layer "F.Cu") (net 11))
 (segment (start 113.03 82.55) (end 113.03 97.79) (width 0.2) (layer "F.Cu") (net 11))
 (segment (start 212.486228 17.280615) (end 212.486228 160.790615) (width 0.2) (layer "F.Cu") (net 17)))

